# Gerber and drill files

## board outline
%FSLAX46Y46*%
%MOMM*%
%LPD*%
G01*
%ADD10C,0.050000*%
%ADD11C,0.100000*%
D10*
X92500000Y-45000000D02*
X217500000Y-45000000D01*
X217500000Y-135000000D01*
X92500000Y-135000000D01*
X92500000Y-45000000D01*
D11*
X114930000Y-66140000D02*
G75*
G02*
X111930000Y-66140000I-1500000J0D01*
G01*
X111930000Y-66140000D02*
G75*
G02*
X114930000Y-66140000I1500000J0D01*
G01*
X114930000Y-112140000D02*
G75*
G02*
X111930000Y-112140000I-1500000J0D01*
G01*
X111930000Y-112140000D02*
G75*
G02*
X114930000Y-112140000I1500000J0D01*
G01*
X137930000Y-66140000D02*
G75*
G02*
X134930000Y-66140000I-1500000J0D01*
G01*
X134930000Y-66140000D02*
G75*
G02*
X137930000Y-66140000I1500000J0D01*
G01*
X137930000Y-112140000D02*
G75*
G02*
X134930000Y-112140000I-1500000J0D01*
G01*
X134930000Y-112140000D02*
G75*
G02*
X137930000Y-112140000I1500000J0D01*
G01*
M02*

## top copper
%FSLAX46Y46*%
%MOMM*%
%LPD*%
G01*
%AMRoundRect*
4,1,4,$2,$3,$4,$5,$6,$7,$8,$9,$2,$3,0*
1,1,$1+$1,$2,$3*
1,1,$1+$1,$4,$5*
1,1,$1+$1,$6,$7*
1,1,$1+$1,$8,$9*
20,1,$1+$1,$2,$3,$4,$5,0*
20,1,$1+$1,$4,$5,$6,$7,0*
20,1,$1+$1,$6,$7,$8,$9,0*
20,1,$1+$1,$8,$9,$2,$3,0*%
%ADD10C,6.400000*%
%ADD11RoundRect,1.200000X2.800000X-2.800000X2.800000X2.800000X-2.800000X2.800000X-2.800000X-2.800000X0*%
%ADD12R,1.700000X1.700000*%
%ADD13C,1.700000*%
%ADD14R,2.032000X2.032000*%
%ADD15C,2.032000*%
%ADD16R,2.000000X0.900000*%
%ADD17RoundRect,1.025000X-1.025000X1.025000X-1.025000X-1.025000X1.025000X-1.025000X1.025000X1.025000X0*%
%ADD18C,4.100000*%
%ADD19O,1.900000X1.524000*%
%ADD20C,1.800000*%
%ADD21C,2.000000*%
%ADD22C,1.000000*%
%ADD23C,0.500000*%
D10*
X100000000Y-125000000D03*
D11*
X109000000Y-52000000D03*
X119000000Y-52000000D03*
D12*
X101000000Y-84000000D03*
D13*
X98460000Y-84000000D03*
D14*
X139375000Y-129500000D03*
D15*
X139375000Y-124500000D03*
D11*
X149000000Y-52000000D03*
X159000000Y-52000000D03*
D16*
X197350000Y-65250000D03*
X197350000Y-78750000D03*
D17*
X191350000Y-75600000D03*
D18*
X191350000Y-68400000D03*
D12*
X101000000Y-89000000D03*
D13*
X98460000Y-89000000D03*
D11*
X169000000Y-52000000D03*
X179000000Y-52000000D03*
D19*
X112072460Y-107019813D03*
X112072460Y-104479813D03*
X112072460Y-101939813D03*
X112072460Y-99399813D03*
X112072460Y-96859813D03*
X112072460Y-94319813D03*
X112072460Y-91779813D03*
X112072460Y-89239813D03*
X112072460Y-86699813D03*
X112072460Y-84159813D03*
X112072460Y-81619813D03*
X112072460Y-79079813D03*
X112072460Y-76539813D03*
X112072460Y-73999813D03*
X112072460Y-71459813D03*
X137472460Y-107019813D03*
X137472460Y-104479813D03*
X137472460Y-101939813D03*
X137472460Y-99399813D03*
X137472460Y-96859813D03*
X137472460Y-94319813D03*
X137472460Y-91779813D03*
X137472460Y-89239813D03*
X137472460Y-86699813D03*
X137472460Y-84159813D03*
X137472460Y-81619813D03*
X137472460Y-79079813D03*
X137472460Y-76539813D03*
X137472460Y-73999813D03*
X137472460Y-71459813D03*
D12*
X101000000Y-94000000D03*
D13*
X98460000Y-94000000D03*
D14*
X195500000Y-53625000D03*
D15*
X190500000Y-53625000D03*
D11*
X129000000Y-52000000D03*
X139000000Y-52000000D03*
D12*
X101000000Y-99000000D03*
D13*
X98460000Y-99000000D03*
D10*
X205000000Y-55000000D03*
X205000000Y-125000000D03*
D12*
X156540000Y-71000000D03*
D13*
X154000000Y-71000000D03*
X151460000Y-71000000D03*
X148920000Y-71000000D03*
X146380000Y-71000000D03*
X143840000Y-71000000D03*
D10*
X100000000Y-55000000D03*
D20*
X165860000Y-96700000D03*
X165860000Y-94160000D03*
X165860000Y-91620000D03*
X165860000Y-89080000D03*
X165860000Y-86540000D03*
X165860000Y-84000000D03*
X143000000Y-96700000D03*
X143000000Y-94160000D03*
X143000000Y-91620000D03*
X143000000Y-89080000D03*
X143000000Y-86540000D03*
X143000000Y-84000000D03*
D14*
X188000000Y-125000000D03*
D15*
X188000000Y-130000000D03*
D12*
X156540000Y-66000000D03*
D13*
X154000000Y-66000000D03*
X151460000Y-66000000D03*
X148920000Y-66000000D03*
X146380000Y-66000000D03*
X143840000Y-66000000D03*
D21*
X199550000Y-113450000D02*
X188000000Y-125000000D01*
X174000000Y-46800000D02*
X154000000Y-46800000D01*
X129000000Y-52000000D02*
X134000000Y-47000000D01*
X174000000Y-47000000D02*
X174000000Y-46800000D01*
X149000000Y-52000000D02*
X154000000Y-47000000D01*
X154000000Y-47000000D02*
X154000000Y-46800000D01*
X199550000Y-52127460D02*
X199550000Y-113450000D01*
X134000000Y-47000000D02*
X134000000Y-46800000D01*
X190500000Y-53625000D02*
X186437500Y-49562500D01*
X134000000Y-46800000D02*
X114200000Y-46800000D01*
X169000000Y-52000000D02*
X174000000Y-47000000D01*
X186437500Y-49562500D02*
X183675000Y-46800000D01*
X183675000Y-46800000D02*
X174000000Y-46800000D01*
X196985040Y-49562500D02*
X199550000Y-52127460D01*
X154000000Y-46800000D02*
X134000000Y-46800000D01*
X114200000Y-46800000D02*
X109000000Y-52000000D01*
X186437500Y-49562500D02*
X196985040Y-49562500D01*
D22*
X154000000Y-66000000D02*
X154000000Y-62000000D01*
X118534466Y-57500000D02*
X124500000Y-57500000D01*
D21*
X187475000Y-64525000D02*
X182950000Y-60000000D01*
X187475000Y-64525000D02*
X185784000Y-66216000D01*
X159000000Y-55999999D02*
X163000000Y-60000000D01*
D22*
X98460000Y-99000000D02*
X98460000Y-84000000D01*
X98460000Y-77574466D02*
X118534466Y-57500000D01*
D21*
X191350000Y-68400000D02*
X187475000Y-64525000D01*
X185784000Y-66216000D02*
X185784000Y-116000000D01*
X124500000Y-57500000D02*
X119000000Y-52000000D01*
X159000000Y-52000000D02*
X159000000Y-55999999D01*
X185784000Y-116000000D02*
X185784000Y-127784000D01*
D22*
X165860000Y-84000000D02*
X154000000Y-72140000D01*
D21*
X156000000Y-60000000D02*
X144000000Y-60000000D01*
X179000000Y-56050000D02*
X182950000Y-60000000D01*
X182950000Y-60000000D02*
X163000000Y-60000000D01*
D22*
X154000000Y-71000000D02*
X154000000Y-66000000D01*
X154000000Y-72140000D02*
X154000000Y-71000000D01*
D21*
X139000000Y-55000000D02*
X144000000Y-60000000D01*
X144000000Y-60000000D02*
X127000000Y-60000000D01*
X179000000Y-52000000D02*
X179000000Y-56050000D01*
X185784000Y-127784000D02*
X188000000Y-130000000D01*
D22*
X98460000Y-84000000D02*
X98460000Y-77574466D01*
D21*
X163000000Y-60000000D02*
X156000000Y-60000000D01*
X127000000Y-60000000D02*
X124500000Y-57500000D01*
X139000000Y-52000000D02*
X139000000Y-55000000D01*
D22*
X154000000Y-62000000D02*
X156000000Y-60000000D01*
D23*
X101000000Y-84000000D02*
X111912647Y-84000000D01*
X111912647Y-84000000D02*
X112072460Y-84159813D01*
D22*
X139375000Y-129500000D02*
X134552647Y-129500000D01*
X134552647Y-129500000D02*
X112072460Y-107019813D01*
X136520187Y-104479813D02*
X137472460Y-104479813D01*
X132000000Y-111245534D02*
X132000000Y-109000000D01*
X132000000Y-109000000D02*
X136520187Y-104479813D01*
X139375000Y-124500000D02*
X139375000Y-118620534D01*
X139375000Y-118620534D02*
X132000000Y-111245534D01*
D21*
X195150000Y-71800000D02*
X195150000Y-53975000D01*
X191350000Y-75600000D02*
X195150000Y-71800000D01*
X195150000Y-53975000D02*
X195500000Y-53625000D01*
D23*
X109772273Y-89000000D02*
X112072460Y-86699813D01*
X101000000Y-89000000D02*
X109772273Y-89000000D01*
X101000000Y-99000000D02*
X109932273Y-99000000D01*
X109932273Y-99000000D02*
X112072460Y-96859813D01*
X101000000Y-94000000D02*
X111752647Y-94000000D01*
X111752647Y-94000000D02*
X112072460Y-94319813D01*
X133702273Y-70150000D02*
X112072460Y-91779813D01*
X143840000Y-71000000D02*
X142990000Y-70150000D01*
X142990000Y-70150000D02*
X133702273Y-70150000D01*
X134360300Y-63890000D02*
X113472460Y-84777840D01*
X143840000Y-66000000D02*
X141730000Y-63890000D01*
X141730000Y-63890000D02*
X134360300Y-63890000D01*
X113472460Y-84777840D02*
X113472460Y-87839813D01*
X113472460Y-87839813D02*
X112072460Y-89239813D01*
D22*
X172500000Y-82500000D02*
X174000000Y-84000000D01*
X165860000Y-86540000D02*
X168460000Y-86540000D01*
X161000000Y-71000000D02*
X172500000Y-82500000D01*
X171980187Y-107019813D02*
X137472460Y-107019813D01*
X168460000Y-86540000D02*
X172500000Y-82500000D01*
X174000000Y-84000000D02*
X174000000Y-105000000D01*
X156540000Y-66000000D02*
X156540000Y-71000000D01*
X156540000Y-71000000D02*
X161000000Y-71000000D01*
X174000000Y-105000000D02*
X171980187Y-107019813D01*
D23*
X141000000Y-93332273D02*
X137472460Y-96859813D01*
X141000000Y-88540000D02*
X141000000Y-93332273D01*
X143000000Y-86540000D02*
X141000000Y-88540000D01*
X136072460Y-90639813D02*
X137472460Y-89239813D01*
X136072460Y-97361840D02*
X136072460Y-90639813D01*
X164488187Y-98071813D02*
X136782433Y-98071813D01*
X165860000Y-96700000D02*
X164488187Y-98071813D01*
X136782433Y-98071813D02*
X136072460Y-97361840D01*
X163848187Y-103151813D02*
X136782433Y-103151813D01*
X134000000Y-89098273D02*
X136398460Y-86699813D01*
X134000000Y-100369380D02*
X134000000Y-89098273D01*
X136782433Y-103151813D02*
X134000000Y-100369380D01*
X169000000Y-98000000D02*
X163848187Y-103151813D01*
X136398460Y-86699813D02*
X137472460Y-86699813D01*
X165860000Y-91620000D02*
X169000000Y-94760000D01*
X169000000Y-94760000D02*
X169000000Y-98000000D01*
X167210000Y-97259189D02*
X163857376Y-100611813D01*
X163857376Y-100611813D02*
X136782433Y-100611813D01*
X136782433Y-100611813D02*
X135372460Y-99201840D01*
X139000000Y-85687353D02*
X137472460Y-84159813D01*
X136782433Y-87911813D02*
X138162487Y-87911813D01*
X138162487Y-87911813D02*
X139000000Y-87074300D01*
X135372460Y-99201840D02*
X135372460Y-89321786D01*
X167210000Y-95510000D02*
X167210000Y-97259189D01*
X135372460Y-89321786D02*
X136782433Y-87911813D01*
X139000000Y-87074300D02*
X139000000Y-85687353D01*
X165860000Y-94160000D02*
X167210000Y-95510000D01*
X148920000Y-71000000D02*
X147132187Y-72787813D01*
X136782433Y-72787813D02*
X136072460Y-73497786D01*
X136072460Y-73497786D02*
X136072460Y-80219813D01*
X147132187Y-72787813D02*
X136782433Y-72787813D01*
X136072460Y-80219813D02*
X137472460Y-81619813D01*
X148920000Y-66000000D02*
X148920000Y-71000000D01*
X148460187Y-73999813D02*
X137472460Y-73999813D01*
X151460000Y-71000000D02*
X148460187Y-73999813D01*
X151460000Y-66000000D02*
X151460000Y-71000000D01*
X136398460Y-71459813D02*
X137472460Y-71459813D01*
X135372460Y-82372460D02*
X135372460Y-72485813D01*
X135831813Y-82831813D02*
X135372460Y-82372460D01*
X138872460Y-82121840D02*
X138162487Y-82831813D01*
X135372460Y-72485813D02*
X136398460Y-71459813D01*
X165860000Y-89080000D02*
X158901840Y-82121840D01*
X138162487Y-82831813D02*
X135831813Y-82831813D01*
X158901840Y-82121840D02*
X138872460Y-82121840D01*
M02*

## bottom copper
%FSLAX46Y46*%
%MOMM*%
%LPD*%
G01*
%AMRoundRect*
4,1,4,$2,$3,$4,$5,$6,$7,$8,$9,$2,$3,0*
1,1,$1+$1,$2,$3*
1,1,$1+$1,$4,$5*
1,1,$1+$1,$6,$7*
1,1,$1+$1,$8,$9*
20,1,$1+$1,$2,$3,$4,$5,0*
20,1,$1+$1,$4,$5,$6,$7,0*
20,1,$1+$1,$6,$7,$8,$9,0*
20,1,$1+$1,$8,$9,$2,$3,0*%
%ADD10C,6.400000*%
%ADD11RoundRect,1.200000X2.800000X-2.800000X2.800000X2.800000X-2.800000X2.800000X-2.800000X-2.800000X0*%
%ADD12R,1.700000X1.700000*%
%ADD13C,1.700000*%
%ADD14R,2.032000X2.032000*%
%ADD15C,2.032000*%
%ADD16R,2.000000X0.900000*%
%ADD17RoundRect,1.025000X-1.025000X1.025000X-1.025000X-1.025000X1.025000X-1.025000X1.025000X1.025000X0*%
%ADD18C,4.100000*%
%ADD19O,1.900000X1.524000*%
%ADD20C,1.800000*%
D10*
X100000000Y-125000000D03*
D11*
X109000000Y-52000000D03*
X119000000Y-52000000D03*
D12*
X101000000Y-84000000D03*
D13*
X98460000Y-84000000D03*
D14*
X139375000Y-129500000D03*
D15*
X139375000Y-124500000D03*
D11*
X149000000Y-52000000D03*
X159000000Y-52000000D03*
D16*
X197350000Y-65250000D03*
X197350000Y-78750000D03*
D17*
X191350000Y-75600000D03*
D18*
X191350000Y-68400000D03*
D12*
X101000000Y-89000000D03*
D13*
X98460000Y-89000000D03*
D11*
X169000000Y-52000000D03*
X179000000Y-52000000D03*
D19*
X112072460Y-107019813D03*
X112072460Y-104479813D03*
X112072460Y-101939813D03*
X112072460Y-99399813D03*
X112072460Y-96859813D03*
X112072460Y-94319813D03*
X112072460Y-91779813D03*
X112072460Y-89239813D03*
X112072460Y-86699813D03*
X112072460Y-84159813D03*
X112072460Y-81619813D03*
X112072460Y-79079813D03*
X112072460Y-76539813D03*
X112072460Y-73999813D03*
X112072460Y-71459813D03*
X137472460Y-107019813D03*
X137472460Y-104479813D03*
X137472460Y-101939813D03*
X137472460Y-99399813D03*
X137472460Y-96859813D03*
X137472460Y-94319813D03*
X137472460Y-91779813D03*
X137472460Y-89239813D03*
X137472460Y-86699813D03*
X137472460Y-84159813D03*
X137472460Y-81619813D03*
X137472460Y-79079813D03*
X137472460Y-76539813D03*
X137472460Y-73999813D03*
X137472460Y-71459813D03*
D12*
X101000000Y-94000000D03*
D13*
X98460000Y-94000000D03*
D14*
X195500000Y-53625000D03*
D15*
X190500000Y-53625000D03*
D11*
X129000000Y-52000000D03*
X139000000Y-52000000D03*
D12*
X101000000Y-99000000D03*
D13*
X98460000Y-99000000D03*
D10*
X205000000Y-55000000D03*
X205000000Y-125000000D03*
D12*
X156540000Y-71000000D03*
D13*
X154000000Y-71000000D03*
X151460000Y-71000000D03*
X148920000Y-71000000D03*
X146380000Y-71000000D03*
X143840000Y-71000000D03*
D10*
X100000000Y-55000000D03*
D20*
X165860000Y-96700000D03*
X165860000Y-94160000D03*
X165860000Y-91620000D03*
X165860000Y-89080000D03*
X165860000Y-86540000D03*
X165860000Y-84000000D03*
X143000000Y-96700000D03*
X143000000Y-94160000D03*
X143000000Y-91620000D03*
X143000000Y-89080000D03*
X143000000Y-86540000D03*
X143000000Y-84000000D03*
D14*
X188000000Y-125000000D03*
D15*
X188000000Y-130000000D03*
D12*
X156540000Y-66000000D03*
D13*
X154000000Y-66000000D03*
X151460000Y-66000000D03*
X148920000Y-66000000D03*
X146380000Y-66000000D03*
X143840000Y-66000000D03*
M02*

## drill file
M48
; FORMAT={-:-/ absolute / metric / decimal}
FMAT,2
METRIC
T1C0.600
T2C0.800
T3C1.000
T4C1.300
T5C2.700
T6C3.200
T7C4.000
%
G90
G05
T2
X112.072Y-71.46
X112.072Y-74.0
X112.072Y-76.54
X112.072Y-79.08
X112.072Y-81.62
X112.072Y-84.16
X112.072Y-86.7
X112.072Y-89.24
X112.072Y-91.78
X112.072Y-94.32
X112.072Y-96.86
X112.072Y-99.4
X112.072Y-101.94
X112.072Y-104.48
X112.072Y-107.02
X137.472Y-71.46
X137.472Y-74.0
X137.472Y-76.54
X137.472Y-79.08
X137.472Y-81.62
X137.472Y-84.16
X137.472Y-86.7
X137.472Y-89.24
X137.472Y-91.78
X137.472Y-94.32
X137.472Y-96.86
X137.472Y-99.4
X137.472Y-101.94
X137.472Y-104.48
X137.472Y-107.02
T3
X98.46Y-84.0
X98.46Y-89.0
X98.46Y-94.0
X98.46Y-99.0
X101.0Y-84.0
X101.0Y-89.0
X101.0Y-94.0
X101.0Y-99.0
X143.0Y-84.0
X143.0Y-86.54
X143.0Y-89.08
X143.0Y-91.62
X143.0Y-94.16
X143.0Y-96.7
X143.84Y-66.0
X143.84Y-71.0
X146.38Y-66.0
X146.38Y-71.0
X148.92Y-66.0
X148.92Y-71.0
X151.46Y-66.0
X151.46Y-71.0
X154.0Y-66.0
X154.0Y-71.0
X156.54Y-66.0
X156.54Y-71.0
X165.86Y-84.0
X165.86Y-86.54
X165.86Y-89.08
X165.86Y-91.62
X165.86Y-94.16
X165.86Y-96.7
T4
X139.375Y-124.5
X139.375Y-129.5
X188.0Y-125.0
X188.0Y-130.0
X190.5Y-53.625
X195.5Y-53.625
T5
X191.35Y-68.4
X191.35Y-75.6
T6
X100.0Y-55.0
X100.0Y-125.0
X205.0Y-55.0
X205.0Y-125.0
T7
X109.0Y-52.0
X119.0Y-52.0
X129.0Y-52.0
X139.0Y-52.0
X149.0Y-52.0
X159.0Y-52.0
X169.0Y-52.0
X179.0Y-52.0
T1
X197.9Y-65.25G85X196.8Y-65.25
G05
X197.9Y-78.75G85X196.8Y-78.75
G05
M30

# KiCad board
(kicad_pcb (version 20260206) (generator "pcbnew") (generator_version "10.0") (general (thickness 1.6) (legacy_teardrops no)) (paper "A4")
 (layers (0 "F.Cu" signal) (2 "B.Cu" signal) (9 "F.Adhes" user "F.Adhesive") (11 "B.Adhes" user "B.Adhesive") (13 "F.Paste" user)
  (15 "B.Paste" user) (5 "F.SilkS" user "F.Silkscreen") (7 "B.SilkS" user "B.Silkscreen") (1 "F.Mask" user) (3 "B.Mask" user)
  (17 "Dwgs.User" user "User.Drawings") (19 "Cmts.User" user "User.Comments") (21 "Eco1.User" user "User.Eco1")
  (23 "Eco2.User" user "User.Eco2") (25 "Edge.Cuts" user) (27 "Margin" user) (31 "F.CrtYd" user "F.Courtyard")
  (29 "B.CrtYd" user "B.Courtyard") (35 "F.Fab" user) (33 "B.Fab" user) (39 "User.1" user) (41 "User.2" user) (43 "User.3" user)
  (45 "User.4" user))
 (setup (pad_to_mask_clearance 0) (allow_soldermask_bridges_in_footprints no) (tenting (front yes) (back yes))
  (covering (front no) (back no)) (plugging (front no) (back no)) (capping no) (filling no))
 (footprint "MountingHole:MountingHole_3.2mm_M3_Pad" (layer "F.Cu") (at 100 125)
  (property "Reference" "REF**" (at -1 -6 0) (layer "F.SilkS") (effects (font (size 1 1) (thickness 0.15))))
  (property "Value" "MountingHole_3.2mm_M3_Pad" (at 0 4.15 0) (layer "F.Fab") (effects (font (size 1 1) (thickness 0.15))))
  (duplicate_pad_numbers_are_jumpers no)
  (pad "1" thru_hole circle (at 0 0) (size 6.4 6.4) (drill 3.2) (layers "*.Cu" "*.Mask") (remove_unused_layers no) (zone_connect 2)))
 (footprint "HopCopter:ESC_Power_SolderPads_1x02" (layer "F.Cu") (at 114 52)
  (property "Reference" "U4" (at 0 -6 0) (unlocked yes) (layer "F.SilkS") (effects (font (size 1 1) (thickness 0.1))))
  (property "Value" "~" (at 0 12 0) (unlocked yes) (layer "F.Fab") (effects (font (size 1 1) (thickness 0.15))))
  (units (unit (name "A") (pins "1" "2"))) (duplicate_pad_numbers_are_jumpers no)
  (pad "1" thru_hole roundrect (at -5 0 90) (size 8 8) (drill 4) (layers "*.Cu" "*.Mask") (remove_unused_layers no) (roundrect_rratio 0.15)
   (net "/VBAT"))
  (pad "2" thru_hole roundrect (at 5 0 90) (size 8 8) (drill 4) (layers "*.Cu" "*.Mask") (remove_unused_layers no) (roundrect_rratio 0.15)
   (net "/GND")))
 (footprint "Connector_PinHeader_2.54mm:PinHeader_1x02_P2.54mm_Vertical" (layer "F.Cu") (at 101 84 -90)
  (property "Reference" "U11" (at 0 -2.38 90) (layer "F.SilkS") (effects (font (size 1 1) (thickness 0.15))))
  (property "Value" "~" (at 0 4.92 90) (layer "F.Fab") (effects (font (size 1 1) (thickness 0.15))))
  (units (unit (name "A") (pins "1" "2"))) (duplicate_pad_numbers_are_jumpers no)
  (pad "1" thru_hole rect (at 0 0 270) (size 1.7 1.7) (drill 1) (layers "*.Cu" "*.Mask") (remove_unused_layers no) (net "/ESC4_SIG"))
  (pad "2" thru_hole circle (at 0 2.54 270) (size 1.7 1.7) (drill 1) (layers "*.Cu" "*.Mask") (remove_unused_layers no) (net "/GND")))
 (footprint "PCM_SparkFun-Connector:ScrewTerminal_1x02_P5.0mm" (layer "F.Cu") (at 139.375 129.5 90)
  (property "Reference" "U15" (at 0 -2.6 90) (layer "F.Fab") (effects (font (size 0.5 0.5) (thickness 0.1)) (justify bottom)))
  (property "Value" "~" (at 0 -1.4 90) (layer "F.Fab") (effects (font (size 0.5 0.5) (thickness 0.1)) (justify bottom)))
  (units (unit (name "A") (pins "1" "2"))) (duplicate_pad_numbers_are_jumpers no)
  (pad "1" thru_hole rect (at 0 0 90) (size 2.032 2.032) (drill 1.3) (layers "*.Cu" "*.Mask") (remove_unused_layers no)
   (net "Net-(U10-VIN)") (thermal_bridge_angle 0))
  (pad "2" thru_hole circle (at 5 0 90) (size 2.032 2.032) (drill 1.3) (layers "*.Cu" "*.Mask") (remove_unused_layers no)
   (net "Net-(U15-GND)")))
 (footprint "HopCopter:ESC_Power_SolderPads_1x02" (layer "F.Cu") (at 154 52)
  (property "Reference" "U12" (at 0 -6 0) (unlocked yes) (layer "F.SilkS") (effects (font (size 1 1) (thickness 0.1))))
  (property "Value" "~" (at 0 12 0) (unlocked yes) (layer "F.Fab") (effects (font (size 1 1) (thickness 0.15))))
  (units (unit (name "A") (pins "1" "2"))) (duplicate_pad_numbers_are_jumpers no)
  (pad "1" thru_hole roundrect (at -5 0 90) (size 8 8) (drill 4) (layers "*.Cu" "*.Mask") (remove_unused_layers no) (roundrect_rratio 0.15)
   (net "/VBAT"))
  (pad "2" thru_hole roundrect (at 5 0 90) (size 8 8) (drill 4) (layers "*.Cu" "*.Mask") (remove_unused_layers no) (roundrect_rratio 0.15)
   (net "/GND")))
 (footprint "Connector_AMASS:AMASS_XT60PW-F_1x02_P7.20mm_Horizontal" (layer "F.Cu") (at 191.35 75.6 -90)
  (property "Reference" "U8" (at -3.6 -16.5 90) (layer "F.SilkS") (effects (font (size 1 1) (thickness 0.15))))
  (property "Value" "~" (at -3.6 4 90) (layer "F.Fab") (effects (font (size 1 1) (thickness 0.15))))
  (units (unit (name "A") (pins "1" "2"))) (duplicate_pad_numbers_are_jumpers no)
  (pad "" thru_hole rect (at -10.35 -6 270) (size 0.9 2) (drill oval 0.6 1.7) (layers "*.Cu" "*.Mask") (remove_unused_layers no))
  (pad "" thru_hole rect (at 3.15 -6 270) (size 0.9 2) (drill oval 0.6 1.7) (layers "*.Cu" "*.Mask") (remove_unused_layers no))
  (pad "1" thru_hole roundrect (at 0 0 270) (size 4.1 4.1) (drill 2.7) (layers "*.Cu" "*.Mask") (remove_unused_layers no)
   (roundrect_rratio 0.25) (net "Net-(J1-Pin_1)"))
  (pad "2" thru_hole circle (at -7.2 0 270) (size 4.1 4.1) (drill 2.7) (layers "*.Cu" "*.Mask") (remove_unused_layers no) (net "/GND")))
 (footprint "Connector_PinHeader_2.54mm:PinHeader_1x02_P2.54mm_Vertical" (layer "F.Cu") (at 101 89 -90)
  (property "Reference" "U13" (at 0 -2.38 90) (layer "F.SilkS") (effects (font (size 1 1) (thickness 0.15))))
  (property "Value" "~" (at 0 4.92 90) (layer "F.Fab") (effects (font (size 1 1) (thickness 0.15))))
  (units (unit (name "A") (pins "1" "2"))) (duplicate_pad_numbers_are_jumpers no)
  (pad "1" thru_hole rect (at 0 0 270) (size 1.7 1.7) (drill 1) (layers "*.Cu" "*.Mask") (remove_unused_layers no) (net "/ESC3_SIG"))
  (pad "2" thru_hole circle (at 0 2.54 270) (size 1.7 1.7) (drill 1) (layers "*.Cu" "*.Mask") (remove_unused_layers no) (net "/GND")))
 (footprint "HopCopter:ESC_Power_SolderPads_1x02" (layer "F.Cu") (at 174 52)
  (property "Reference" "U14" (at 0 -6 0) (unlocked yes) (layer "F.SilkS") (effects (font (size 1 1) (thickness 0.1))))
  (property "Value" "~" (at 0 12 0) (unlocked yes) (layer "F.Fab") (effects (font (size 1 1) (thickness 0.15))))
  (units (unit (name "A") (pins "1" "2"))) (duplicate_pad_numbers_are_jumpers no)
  (pad "1" thru_hole roundrect (at -5 0 90) (size 8 8) (drill 4) (layers "*.Cu" "*.Mask") (remove_unused_layers no) (roundrect_rratio 0.15)
   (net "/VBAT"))
  (pad "2" thru_hole roundrect (at 5 0 90) (size 8 8) (drill 4) (layers "*.Cu" "*.Mask") (remove_unused_layers no) (roundrect_rratio 0.15)
   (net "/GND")))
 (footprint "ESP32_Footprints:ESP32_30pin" (layer "F.Cu") (at 124 90)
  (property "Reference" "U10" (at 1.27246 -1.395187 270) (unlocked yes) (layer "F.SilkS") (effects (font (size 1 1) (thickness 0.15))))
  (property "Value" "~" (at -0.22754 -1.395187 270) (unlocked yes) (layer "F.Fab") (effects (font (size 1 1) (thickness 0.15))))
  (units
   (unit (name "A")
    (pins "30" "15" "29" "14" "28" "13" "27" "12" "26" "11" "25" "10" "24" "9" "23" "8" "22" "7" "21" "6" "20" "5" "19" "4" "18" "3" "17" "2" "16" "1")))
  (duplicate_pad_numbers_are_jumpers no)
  (fp_circle (center -10.57 -23.86) (end -10.57 -22.36) (stroke (width 0.1) (type default)) (fill no) (layer "Edge.Cuts"))
  (fp_circle (center -10.57 22.14) (end -10.57 23.64) (stroke (width 0.1) (type default)) (fill no) (layer "Edge.Cuts"))
  (fp_circle (center 12.43 -23.86) (end 12.43 -22.36) (stroke (width 0.1) (type default)) (fill no) (layer "Edge.Cuts"))
  (fp_circle (center 12.43 22.14) (end 12.43 23.64) (stroke (width 0.1) (type default)) (fill no) (layer "Edge.Cuts"))
  (pad "1" thru_hole oval (at -11.92754 17.019813 270) (size 1.524 1.9) (drill 0.8) (layers "*.Cu" "*.Mask") (remove_unused_layers no)
   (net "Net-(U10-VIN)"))
  (pad "2" thru_hole oval (at -11.92754 14.479813 270) (size 1.524 1.9) (drill 0.8) (layers "*.Cu" "*.Mask") (remove_unused_layers no)
   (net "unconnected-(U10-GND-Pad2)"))
  (pad "3" thru_hole oval (at -11.92754 11.939813 270) (size 1.524 1.9) (drill 0.8) (layers "*.Cu" "*.Mask") (remove_unused_layers no)
   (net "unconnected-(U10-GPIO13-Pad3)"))
  (pad "4" thru_hole oval (at -11.92754 9.399813 270) (size 1.524 1.9) (drill 0.8) (layers "*.Cu" "*.Mask") (remove_unused_layers no)
   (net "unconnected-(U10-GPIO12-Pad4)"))
  (pad "5" thru_hole oval (at -11.92754 6.859813 270) (size 1.524 1.9) (drill 0.8) (layers "*.Cu" "*.Mask") (remove_unused_layers no)
   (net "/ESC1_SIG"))
  (pad "6" thru_hole oval (at -11.92754 4.319813 270) (size 1.524 1.9) (drill 0.8) (layers "*.Cu" "*.Mask") (remove_unused_layers no)
   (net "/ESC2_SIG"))
  (pad "7" thru_hole oval (at -11.92754 1.779813 270) (size 1.524 1.9) (drill 0.8) (layers "*.Cu" "*.Mask") (remove_unused_layers no)
   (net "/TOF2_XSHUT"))
  (pad "8" thru_hole oval (at -11.92754 -0.760187 270) (size 1.524 1.9) (drill 0.8) (layers "*.Cu" "*.Mask") (remove_unused_layers no)
   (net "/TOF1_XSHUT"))
  (pad "9" thru_hole oval (at -11.92754 -3.300187 270) (size 1.524 1.9) (drill 0.8) (layers "*.Cu" "*.Mask") (remove_unused_layers no)
   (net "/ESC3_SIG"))
  (pad "10" thru_hole oval (at -11.92754 -5.840187 270) (size 1.524 1.9) (drill 0.8) (layers "*.Cu" "*.Mask") (remove_unused_layers no)
   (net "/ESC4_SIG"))
  (pad "11" thru_hole oval (at -11.92754 -8.380187 270) (size 1.524 1.9) (drill 0.8) (layers "*.Cu" "*.Mask") (remove_unused_layers no)
   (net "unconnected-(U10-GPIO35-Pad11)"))
  (pad "12" thru_hole oval (at -11.92754 -10.920187 270) (size 1.524 1.9) (drill 0.8) (layers "*.Cu" "*.Mask") (remove_unused_layers no)
   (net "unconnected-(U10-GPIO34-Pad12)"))
  (pad "13" thru_hole oval (at -11.92754 -13.460187 270) (size 1.524 1.9) (drill 0.8) (layers "*.Cu" "*.Mask") (remove_unused_layers no)
   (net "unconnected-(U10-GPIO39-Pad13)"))
  (pad "14" thru_hole oval (at -11.92754 -16.000187 270) (size 1.524 1.9) (drill 0.8) (layers "*.Cu" "*.Mask") (remove_unused_layers no)
   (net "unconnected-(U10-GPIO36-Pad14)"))
  (pad "15" thru_hole oval (at -11.92754 -18.540187 270) (size 1.524 1.9) (drill 0.8) (layers "*.Cu" "*.Mask") (remove_unused_layers no)
   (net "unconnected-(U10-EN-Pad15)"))
  (pad "16" thru_hole oval (at 13.47246 17.019813 270) (size 1.524 1.9) (drill 0.8) (layers "*.Cu" "*.Mask") (remove_unused_layers no)
   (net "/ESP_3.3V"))
  (pad "17" thru_hole oval (at 13.47246 14.479813 270) (size 1.524 1.9) (drill 0.8) (layers "*.Cu" "*.Mask") (remove_unused_layers no)
   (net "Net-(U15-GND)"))
  (pad "18" thru_hole oval (at 13.47246 11.939813 270) (size 1.524 1.9) (drill 0.8) (layers "*.Cu" "*.Mask") (remove_unused_layers no)
   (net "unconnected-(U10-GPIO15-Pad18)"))
  (pad "19" thru_hole oval (at 13.47246 9.399813 270) (size 1.524 1.9) (drill 0.8) (layers "*.Cu" "*.Mask") (remove_unused_layers no)
   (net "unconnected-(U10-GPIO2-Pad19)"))
  (pad "20" thru_hole oval (at 13.47246 6.859813 270) (size 1.524 1.9) (drill 0.8) (layers "*.Cu" "*.Mask" "Dwgs.User")
   (remove_unused_layers no) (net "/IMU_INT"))
  (pad "21" thru_hole oval (at 13.47246 4.319813 270) (size 1.524 1.9) (drill 0.8) (layers "*.Cu" "*.Mask") (remove_unused_layers no)
   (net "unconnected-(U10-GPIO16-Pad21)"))
  (pad "22" thru_hole oval (at 13.47246 1.779813 270) (size 1.524 1.9) (drill 0.8) (layers "*.Cu" "*.Mask") (remove_unused_layers no)
   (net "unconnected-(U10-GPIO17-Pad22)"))
  (pad "23" thru_hole oval (at 13.47246 -0.760187 270) (size 1.524 1.9) (drill 0.8) (layers "*.Cu" "*.Mask") (remove_unused_layers no)
   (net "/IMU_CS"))
  (pad "24" thru_hole oval (at 13.47246 -3.300187 270) (size 1.524 1.9) (drill 0.8) (layers "*.Cu" "*.Mask") (remove_unused_layers no)
   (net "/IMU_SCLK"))
  (pad "25" thru_hole oval (at 13.47246 -5.840187 270) (size 1.524 1.9) (drill 0.8) (layers "*.Cu" "*.Mask") (remove_unused_layers no)
   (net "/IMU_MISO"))
  (pad "26" thru_hole oval (at 13.47246 -8.380187 270) (size 1.524 1.9) (drill 0.8) (layers "*.Cu" "*.Mask") (remove_unused_layers no)
   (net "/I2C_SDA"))
  (pad "27" thru_hole oval (at 13.47246 -10.920187 270) (size 1.524 1.9) (drill 0.8) (layers "*.Cu" "*.Mask") (remove_unused_layers no)
   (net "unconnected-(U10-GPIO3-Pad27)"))
  (pad "28" thru_hole oval (at 13.47246 -13.460187 270) (size 1.524 1.9) (drill 0.8) (layers "*.Cu" "*.Mask") (remove_unused_layers no)
   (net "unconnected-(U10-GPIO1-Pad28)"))
  (pad "29" thru_hole oval (at 13.47246 -16.000187 270) (size 1.524 1.9) (drill 0.8) (layers "*.Cu" "*.Mask") (remove_unused_layers no)
   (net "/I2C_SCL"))
  (pad "30" thru_hole oval (at 13.47246 -18.540187 270) (size 1.524 1.9) (drill 0.8) (layers "*.Cu" "*.Mask") (remove_unused_layers no)
   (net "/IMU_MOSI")))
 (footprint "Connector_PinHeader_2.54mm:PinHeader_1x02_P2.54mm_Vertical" (layer "F.Cu") (at 101 94 -90)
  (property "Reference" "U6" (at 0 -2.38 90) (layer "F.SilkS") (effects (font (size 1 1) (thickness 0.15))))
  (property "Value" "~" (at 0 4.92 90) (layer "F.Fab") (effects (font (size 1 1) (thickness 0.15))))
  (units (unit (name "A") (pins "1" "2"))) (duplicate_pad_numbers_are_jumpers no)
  (pad "1" thru_hole rect (at 0 0 270) (size 1.7 1.7) (drill 1) (layers "*.Cu" "*.Mask") (remove_unused_layers no) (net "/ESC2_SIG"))
  (pad "2" thru_hole circle (at 0 2.54 270) (size 1.7 1.7) (drill 1) (layers "*.Cu" "*.Mask") (remove_unused_layers no) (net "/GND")))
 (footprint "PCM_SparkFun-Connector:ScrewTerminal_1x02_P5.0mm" (layer "F.Cu") (at 195.5 53.625 180)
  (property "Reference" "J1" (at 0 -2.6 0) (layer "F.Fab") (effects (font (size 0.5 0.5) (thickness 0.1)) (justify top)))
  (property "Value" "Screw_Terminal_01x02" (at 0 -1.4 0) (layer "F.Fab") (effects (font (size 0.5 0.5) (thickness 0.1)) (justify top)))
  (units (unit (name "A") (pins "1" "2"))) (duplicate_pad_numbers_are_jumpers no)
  (pad "1" thru_hole rect (at 0 0 180) (size 2.032 2.032) (drill 1.3) (layers "*.Cu" "*.Mask") (remove_unused_layers no)
   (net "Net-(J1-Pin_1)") (thermal_bridge_angle 0))
  (pad "2" thru_hole circle (at 5 0 180) (size 2.032 2.032) (drill 1.3) (layers "*.Cu" "*.Mask") (remove_unused_layers no) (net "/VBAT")))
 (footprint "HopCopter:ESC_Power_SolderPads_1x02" (layer "F.Cu") (at 134 52)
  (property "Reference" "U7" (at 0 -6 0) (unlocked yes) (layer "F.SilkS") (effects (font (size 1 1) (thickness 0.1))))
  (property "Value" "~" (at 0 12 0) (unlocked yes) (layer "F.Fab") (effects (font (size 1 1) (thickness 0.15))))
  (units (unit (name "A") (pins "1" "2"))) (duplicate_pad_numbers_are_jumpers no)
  (pad "1" thru_hole roundrect (at -5 0 90) (size 8 8) (drill 4) (layers "*.Cu" "*.Mask") (remove_unused_layers no) (roundrect_rratio 0.15)
   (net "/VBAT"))
  (pad "2" thru_hole roundrect (at 5 0 90) (size 8 8) (drill 4) (layers "*.Cu" "*.Mask") (remove_unused_layers no) (roundrect_rratio 0.15)
   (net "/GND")))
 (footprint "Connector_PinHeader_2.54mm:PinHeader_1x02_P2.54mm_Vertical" (layer "F.Cu") (at 101 99 -90)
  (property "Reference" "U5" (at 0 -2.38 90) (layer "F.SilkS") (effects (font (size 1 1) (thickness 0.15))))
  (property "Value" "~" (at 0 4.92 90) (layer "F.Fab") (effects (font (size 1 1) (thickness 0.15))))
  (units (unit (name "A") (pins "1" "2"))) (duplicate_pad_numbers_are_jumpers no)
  (pad "1" thru_hole rect (at 0 0 270) (size 1.7 1.7) (drill 1) (layers "*.Cu" "*.Mask") (remove_unused_layers no) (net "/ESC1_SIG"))
  (pad "2" thru_hole circle (at 0 2.54 270) (size 1.7 1.7) (drill 1) (layers "*.Cu" "*.Mask") (remove_unused_layers no) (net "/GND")))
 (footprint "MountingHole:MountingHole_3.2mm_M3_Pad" (layer "F.Cu") (at 205 55)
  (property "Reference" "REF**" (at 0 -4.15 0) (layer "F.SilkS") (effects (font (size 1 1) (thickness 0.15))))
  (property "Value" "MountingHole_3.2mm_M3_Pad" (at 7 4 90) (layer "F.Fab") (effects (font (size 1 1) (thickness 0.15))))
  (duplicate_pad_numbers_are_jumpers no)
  (pad "1" thru_hole circle (at 0 0) (size 6.4 6.4) (drill 3.2) (layers "*.Cu" "*.Mask") (remove_unused_layers no) (zone_connect 2)))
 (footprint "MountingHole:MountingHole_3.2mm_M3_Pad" (layer "F.Cu") (at 205 125)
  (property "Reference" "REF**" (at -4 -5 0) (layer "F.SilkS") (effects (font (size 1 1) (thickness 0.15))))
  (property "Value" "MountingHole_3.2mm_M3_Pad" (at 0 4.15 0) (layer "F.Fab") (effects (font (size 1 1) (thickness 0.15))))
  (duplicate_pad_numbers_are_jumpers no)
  (pad "1" thru_hole circle (at 0 0) (size 6.4 6.4) (drill 3.2) (layers "*.Cu" "*.Mask") (remove_unused_layers no) (zone_connect 2)))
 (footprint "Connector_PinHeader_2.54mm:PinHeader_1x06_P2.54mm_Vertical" (layer "F.Cu") (at 156.54 71 -90)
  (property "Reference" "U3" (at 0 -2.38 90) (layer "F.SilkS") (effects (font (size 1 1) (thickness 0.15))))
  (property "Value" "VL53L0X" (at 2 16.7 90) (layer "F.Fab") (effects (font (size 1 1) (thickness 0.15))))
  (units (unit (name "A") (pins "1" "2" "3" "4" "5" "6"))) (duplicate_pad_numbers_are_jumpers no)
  (pad "1" thru_hole rect (at 0 0 270) (size 1.7 1.7) (drill 1) (layers "*.Cu" "*.Mask") (remove_unused_layers no) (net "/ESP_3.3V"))
  (pad "2" thru_hole circle (at 0 2.54 270) (size 1.7 1.7) (drill 1) (layers "*.Cu" "*.Mask") (remove_unused_layers no) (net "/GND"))
  (pad "3" thru_hole circle (at 0 5.08 270) (size 1.7 1.7) (drill 1) (layers "*.Cu" "*.Mask") (remove_unused_layers no) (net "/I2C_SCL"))
  (pad "4" thru_hole circle (at 0 7.62 270) (size 1.7 1.7) (drill 1) (layers "*.Cu" "*.Mask") (remove_unused_layers no) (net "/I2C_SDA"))
  (pad "5" thru_hole circle (at 0 10.16 270) (size 1.7 1.7) (drill 1) (layers "*.Cu" "*.Mask") (remove_unused_layers no)
   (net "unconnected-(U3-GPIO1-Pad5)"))
  (pad "6" thru_hole circle (at 0 12.7 270) (size 1.7 1.7) (drill 1) (layers "*.Cu" "*.Mask") (remove_unused_layers no) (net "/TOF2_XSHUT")))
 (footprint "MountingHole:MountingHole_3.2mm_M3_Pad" (layer "F.Cu") (at 100 55)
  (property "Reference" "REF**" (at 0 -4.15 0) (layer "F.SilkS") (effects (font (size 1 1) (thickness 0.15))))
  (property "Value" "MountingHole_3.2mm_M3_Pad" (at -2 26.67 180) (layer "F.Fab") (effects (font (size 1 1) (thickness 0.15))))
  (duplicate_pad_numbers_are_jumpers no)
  (pad "1" thru_hole circle (at 0 0) (size 6.4 6.4) (drill 3.2) (layers "*.Cu" "*.Mask") (remove_unused_layers no) (zone_connect 2)))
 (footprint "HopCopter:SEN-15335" (layer "F.Cu") (at 165.86 96.7 180)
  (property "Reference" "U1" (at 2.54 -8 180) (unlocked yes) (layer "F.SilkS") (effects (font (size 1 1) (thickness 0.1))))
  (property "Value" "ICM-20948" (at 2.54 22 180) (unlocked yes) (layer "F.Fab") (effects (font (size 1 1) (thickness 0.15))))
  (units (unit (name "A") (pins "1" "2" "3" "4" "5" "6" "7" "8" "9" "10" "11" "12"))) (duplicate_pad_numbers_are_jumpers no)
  (pad "1" thru_hole circle (at 0 0 180) (size 1.8 1.8) (drill 1) (layers "*.Cu" "*.Mask") (remove_unused_layers no) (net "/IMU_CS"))
  (pad "2" thru_hole circle (at 0 2.54 180) (size 1.8 1.8) (drill 1) (layers "*.Cu" "*.Mask" "Eco1.User") (remove_unused_layers no)
   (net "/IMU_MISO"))
  (pad "3" thru_hole circle (at 0 5.08 180) (size 1.8 1.8) (drill 1) (layers "*.Cu" "*.Mask" "Eco1.User") (remove_unused_layers no)
   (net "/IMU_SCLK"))
  (pad "4" thru_hole circle (at 0 7.62 180) (size 1.8 1.8) (drill 1) (layers "*.Cu" "*.Mask" "Eco1.User") (remove_unused_layers no)
   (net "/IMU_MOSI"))
  (pad "5" thru_hole circle (at 0 10.16 180) (size 1.8 1.8) (drill 1) (layers "*.Cu" "*.Mask" "Eco1.User") (remove_unused_layers no)
   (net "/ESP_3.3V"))
  (pad "6" thru_hole circle (at 0 12.7 180) (size 1.8 1.8) (drill 1) (layers "*.Cu" "*.Mask" "Eco1.User") (remove_unused_layers no)
   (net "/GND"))
  (pad "7" thru_hole circle (at 22.86 0 180) (size 1.8 1.8) (drill 1) (layers "*.Cu" "*.Mask") (remove_unused_layers no)
   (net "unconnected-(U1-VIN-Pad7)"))
  (pad "8" thru_hole circle (at 22.86 2.54 180) (size 1.8 1.8) (drill 1) (layers "*.Cu" "*.Mask" "Eco1.User") (remove_unused_layers no)
   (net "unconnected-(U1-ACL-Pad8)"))
  (pad "9" thru_hole circle (at 22.86 5.08 180) (size 1.8 1.8) (drill 1) (layers "*.Cu" "*.Mask" "Eco1.User") (remove_unused_layers no)
   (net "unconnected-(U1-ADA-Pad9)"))
  (pad "10" thru_hole circle (at 22.86 7.62 180) (size 1.8 1.8) (drill 1) (layers "*.Cu" "*.Mask" "Eco1.User") (remove_unused_layers no)
   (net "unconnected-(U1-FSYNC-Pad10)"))
  (pad "11" thru_hole circle (at 22.86 10.16 180) (size 1.8 1.8) (drill 1) (layers "*.Cu" "*.Mask" "Eco1.User") (remove_unused_layers no)
   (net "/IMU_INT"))
  (pad "12" thru_hole circle (at 22.86 12.7 180) (size 1.8 1.8) (drill 1) (layers "*.Cu" "*.Mask" "Eco1.User") (remove_unused_layers no)
   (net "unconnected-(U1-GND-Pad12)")))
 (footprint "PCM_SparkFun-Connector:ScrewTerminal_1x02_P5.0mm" (layer "F.Cu") (at 188 125 -90)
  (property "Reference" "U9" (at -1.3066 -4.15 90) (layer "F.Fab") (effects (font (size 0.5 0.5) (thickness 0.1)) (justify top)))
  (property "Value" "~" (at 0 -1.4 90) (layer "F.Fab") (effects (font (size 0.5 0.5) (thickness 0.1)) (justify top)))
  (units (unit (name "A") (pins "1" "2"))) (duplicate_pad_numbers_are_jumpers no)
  (pad "1" thru_hole rect (at 0 0 270) (size 2.032 2.032) (drill 1.3) (layers "*.Cu" "*.Mask") (remove_unused_layers no) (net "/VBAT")
   (thermal_bridge_angle 0))
  (pad "2" thru_hole circle (at 5 0 270) (size 2.032 2.032) (drill 1.3) (layers "*.Cu" "*.Mask") (remove_unused_layers no) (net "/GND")))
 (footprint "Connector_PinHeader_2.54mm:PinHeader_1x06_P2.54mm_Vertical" (layer "F.Cu") (at 156.54 66 -90)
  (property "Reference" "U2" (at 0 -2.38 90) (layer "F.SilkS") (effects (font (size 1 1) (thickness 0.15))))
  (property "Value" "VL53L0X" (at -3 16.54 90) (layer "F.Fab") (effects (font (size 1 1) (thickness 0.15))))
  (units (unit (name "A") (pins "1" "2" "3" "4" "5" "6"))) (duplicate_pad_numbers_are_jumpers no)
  (pad "1" thru_hole rect (at 0 0 270) (size 1.7 1.7) (drill 1) (layers "*.Cu" "*.Mask") (remove_unused_layers no) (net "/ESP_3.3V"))
  (pad "2" thru_hole circle (at 0 2.54 270) (size 1.7 1.7) (drill 1) (layers "*.Cu" "*.Mask") (remove_unused_layers no) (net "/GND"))
  (pad "3" thru_hole circle (at 0 5.08 270) (size 1.7 1.7) (drill 1) (layers "*.Cu" "*.Mask") (remove_unused_layers no) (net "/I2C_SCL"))
  (pad "4" thru_hole circle (at 0 7.62 270) (size 1.7 1.7) (drill 1) (layers "*.Cu" "*.Mask") (remove_unused_layers no) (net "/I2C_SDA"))
  (pad "5" thru_hole circle (at 0 10.16 270) (size 1.7 1.7) (drill 1) (layers "*.Cu" "*.Mask") (remove_unused_layers no)
   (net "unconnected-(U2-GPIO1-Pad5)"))
  (pad "6" thru_hole circle (at 0 12.7 270) (size 1.7 1.7) (drill 1) (layers "*.Cu" "*.Mask") (remove_unused_layers no) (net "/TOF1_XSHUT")))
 (gr_rect (start 92.5 45) (end 217.5 135) (stroke (width 0.05) (type solid)) (fill no) (layer "Edge.Cuts"))
 (segment (start 199.55 113.45) (end 188 125) (width 2) (layer "F.Cu") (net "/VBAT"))
 (segment (start 174 46.8) (end 154 46.8) (width 2) (layer "F.Cu") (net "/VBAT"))
 (segment (start 129 52) (end 134 47) (width 2) (layer "F.Cu") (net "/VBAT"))
 (segment (start 174 47) (end 174 46.8) (width 2) (layer "F.Cu") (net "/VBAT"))
 (segment (start 149 52) (end 154 47) (width 2) (layer "F.Cu") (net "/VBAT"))
 (segment (start 154 47) (end 154 46.8) (width 2) (layer "F.Cu") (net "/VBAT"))
 (segment (start 199.55 52.12746) (end 199.55 113.45) (width 2) (layer "F.Cu") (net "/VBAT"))
 (segment (start 134 47) (end 134 46.8) (width 2) (layer "F.Cu") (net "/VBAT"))
 (segment (start 190.5 53.625) (end 186.4375 49.5625) (width 2) (layer "F.Cu") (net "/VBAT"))
 (segment (start 134 46.8) (end 114.2 46.8) (width 2) (layer "F.Cu") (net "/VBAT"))
 (segment (start 169 52) (end 174 47) (width 2) (layer "F.Cu") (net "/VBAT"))
 (segment (start 186.4375 49.5625) (end 183.675 46.8) (width 2) (layer "F.Cu") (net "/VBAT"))
 (segment (start 183.675 46.8) (end 174 46.8) (width 2) (layer "F.Cu") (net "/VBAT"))
 (segment (start 196.98504 49.5625) (end 199.55 52.12746) (width 2) (layer "F.Cu") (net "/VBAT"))
 (segment (start 154 46.8) (end 134 46.8) (width 2) (layer "F.Cu") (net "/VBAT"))
 (segment (start 114.2 46.8) (end 109 52) (width 2) (layer "F.Cu") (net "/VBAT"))
 (segment (start 186.4375 49.5625) (end 196.98504 49.5625) (width 2) (layer "F.Cu") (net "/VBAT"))
 (segment (start 154 66) (end 154 62) (width 1) (layer "F.Cu") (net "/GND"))
 (segment (start 118.534466 57.5) (end 124.5 57.5) (width 1) (layer "F.Cu") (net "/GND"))
 (segment (start 187.475 64.525) (end 182.95 60) (width 2) (layer "F.Cu") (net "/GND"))
 (segment (start 187.475 64.525) (end 185.784 66.216) (width 2) (layer "F.Cu") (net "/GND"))
 (segment (start 159 55.999999) (end 163 60) (width 2) (layer "F.Cu") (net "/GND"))
 (segment (start 98.46 99) (end 98.46 84) (width 1) (layer "F.Cu") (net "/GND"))
 (segment (start 98.46 77.574466) (end 118.534466 57.5) (width 1) (layer "F.Cu") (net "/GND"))
 (segment (start 191.35 68.4) (end 187.475 64.525) (width 2) (layer "F.Cu") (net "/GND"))
 (segment (start 185.784 66.216) (end 185.784 116) (width 2) (layer "F.Cu") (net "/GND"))
 (segment (start 124.5 57.5) (end 119 52) (width 2) (layer "F.Cu") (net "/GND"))
 (segment (start 159 52) (end 159 55.999999) (width 2) (layer "F.Cu") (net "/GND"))
 (segment (start 185.784 116) (end 185.784 127.784) (width 2) (layer "F.Cu") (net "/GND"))
 (segment (start 165.86 84) (end 154 72.14) (width 1) (layer "F.Cu") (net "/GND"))
 (segment (start 156 60) (end 144 60) (width 2) (layer "F.Cu") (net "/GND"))
 (segment (start 179 56.05) (end 182.95 60) (width 2) (layer "F.Cu") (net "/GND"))
 (segment (start 182.95 60) (end 163 60) (width 2) (layer "F.Cu") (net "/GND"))
 (segment (start 154 71) (end 154 66) (width 1) (layer "F.Cu") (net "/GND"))
 (segment (start 154 72.14) (end 154 71) (width 1) (layer "F.Cu") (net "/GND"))
 (segment (start 139 55) (end 144 60) (width 2) (layer "F.Cu") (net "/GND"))
 (segment (start 144 60) (end 127 60) (width 2) (layer "F.Cu") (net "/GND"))
 (segment (start 179 52) (end 179 56.05) (width 2) (layer "F.Cu") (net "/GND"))
 (segment (start 185.784 127.784) (end 188 130) (width 2) (layer "F.Cu") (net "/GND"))
 (segment (start 98.46 84) (end 98.46 77.574466) (width 1) (layer "F.Cu") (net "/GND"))
 (segment (start 163 60) (end 156 60) (width 2) (layer "F.Cu") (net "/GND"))
 (segment (start 127 60) (end 124.5 57.5) (width 2) (layer "F.Cu") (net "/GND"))
 (segment (start 139 52) (end 139 55) (width 2) (layer "F.Cu") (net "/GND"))
 (segment (start 154 62) (end 156 60) (width 1) (layer "F.Cu") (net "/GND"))
 (segment (start 101 84) (end 111.912647 84) (width 0.5) (layer "F.Cu") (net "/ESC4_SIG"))
 (segment (start 111.912647 84) (end 112.07246 84.159813) (width 0.5) (layer "F.Cu") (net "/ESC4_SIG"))
 (segment (start 139.375 129.5) (end 134.552647 129.5) (width 1) (layer "F.Cu") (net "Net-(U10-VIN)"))
 (segment (start 134.552647 129.5) (end 112.07246 107.019813) (width 1) (layer "F.Cu") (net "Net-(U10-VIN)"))
 (segment (start 136.520187 104.479813) (end 137.47246 104.479813) (width 1) (layer "F.Cu") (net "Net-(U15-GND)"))
 (segment (start 132 111.245534) (end 132 109) (width 1) (layer "F.Cu") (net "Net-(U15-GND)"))
 (segment (start 132 109) (end 136.520187 104.479813) (width 1) (layer "F.Cu") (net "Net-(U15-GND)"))
 (segment (start 139.375 124.5) (end 139.375 118.620534) (width 1) (layer "F.Cu") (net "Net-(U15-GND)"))
 (segment (start 139.375 118.620534) (end 132 111.245534) (width 1) (layer "F.Cu") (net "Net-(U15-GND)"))
 (segment (start 195.15 71.8) (end 195.15 53.975) (width 2) (layer "F.Cu") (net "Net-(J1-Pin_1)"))
 (segment (start 191.35 75.6) (end 195.15 71.8) (width 2) (layer "F.Cu") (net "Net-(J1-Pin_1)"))
 (segment (start 195.15 53.975) (end 195.5 53.625) (width 2) (layer "F.Cu") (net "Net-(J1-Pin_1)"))
 (segment (start 109.772273 89) (end 112.07246 86.699813) (width 0.5) (layer "F.Cu") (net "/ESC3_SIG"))
 (segment (start 101 89) (end 109.772273 89) (width 0.5) (layer "F.Cu") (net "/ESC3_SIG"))
 (segment (start 101 99) (end 109.932273 99) (width 0.5) (layer "F.Cu") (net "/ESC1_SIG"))
 (segment (start 109.932273 99) (end 112.07246 96.859813) (width 0.5) (layer "F.Cu") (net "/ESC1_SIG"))
 (segment (start 101 94) (end 111.752647 94) (width 0.5) (layer "F.Cu") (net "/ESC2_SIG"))
 (segment (start 111.752647 94) (end 112.07246 94.319813) (width 0.5) (layer "F.Cu") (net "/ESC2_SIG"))
 (segment (start 133.702273 70.15) (end 112.07246 91.779813) (width 0.5) (layer "F.Cu") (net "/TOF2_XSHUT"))
 (segment (start 143.84 71) (end 142.99 70.15) (width 0.5) (layer "F.Cu") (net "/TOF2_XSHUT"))
 (segment (start 142.99 70.15) (end 133.702273 70.15) (width 0.5) (layer "F.Cu") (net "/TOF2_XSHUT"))
 (segment (start 134.3603 63.89) (end 113.47246 84.77784) (width 0.5) (layer "F.Cu") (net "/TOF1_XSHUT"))
 (segment (start 143.84 66) (end 141.73 63.89) (width 0.5) (layer "F.Cu") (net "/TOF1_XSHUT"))
 (segment (start 141.73 63.89) (end 134.3603 63.89) (width 0.5) (layer "F.Cu") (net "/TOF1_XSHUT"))
 (segment (start 113.47246 84.77784) (end 113.47246 87.839813) (width 0.5) (layer "F.Cu") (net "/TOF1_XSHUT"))
 (segment (start 113.47246 87.839813) (end 112.07246 89.239813) (width 0.5) (layer "F.Cu") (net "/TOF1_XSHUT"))
 (segment (start 172.5 82.5) (end 174 84) (width 1) (layer "F.Cu") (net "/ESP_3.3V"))
 (segment (start 165.86 86.54) (end 168.46 86.54) (width 1) (layer "F.Cu") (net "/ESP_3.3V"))
 (segment (start 161 71) (end 172.5 82.5) (width 1) (layer "F.Cu") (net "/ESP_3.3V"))
 (segment (start 171.980187 107.019813) (end 137.47246 107.019813) (width 1) (layer "F.Cu") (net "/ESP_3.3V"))
 (segment (start 168.46 86.54) (end 172.5 82.5) (width 1) (layer "F.Cu") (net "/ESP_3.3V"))
 (segment (start 174 84) (end 174 105) (width 1) (layer "F.Cu") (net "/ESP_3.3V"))
 (segment (start 156.54 66) (end 156.54 71) (width 1) (layer "F.Cu") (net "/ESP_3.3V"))
 (segment (start 156.54 71) (end 161 71) (width 1) (layer "F.Cu") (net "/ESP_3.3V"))
 (segment (start 174 105) (end 171.980187 107.019813) (width 1) (layer "F.Cu") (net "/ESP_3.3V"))
 (segment (start 141 93.332273) (end 137.47246 96.859813) (width 0.5) (layer "F.Cu") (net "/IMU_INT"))
 (segment (start 141 88.54) (end 141 93.332273) (width 0.5) (layer "F.Cu") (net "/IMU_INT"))
 (segment (start 143 86.54) (end 141 88.54) (width 0.5) (layer "F.Cu") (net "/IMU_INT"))
 (segment (start 136.07246 90.639813) (end 137.47246 89.239813) (width 0.5) (layer "F.Cu") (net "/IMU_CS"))
 (segment (start 136.07246 97.36184) (end 136.07246 90.639813) (width 0.5) (layer "F.Cu") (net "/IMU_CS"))
 (segment (start 164.488187 98.071813) (end 136.782433 98.071813) (width 0.5) (layer "F.Cu") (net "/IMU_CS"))
 (segment (start 165.86 96.7) (end 164.488187 98.071813) (width 0.5) (layer "F.Cu") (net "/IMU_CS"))
 (segment (start 136.782433 98.071813) (end 136.07246 97.36184) (width 0.5) (layer "F.Cu") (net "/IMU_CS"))
 (segment (start 163.848187 103.151813) (end 136.782433 103.151813) (width 0.5) (layer "F.Cu") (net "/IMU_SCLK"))
 (segment (start 134 89.098273) (end 136.39846 86.699813) (width 0.5) (layer "F.Cu") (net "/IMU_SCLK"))
 (segment (start 134 100.36938) (end 134 89.098273) (width 0.5) (layer "F.Cu") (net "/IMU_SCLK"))
 (segment (start 136.782433 103.151813) (end 134 100.36938) (width 0.5) (layer "F.Cu") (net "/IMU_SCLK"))
 (segment (start 169 98) (end 163.848187 103.151813) (width 0.5) (layer "F.Cu") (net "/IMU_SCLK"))
 (segment (start 136.39846 86.699813) (end 137.47246 86.699813) (width 0.5) (layer "F.Cu") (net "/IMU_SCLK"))
 (segment (start 165.86 91.62) (end 169 94.76) (width 0.5) (layer "F.Cu") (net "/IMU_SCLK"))
 (segment (start 169 94.76) (end 169 98) (width 0.5) (layer "F.Cu") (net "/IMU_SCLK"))
 (segment (start 167.21 97.259189) (end 163.857376 100.611813) (width 0.5) (layer "F.Cu") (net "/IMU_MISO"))
 (segment (start 163.857376 100.611813) (end 136.782433 100.611813) (width 0.5) (layer "F.Cu") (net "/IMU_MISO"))
 (segment (start 136.782433 100.611813) (end 135.37246 99.20184) (width 0.5) (layer "F.Cu") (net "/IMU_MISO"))
 (segment (start 139 85.687353) (end 137.47246 84.159813) (width 0.5) (layer "F.Cu") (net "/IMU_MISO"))
 (segment (start 136.782433 87.911813) (end 138.162487 87.911813) (width 0.5) (layer "F.Cu") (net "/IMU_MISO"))
 (segment (start 138.162487 87.911813) (end 139 87.0743) (width 0.5) (layer "F.Cu") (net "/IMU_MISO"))
 (segment (start 135.37246 99.20184) (end 135.37246 89.321786) (width 0.5) (layer "F.Cu") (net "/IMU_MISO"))
 (segment (start 167.21 95.51) (end 167.21 97.259189) (width 0.5) (layer "F.Cu") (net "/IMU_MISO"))
 (segment (start 135.37246 89.321786) (end 136.782433 87.911813) (width 0.5) (layer "F.Cu") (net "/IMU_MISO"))
 (segment (start 139 87.0743) (end 139 85.687353) (width 0.5) (layer "F.Cu") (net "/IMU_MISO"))
 (segment (start 165.86 94.16) (end 167.21 95.51) (width 0.5) (layer "F.Cu") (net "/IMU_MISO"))
 (segment (start 148.92 71) (end 147.132187 72.787813) (width 0.5) (layer "F.Cu") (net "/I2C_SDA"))
 (segment (start 136.782433 72.787813) (end 136.07246 73.497786) (width 0.5) (layer "F.Cu") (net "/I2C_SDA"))
 (segment (start 136.07246 73.497786) (end 136.07246 80.219813) (width 0.5) (layer "F.Cu") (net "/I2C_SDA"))
 (segment (start 147.132187 72.787813) (end 136.782433 72.787813) (width 0.5) (layer "F.Cu") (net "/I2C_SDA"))
 (segment (start 136.07246 80.219813) (end 137.47246 81.619813) (width 0.5) (layer "F.Cu") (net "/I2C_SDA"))
 (segment (start 148.92 66) (end 148.92 71) (width 0.5) (layer "F.Cu") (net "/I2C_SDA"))
 (segment (start 148.460187 73.999813) (end 137.47246 73.999813) (width 0.5) (layer "F.Cu") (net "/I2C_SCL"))
 (segment (start 151.46 71) (end 148.460187 73.999813) (width 0.5) (layer "F.Cu") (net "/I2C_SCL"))
 (segment (start 151.46 66) (end 151.46 71) (width 0.5) (layer "F.Cu") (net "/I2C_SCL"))
 (segment (start 136.39846 71.459813) (end 137.47246 71.459813) (width 0.5) (layer "F.Cu") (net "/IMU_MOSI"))
 (segment (start 135.37246 82.37246) (end 135.37246 72.485813) (width 0.5) (layer "F.Cu") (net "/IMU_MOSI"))
 (segment (start 135.831813 82.831813) (end 135.37246 82.37246) (width 0.5) (layer "F.Cu") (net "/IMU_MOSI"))
 (segment (start 138.87246 82.12184) (end 138.162487 82.831813) (width 0.5) (layer "F.Cu") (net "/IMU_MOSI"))
 (segment (start 135.37246 72.485813) (end 136.39846 71.459813) (width 0.5) (layer "F.Cu") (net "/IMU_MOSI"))
 (segment (start 165.86 89.08) (end 158.90184 82.12184) (width 0.5) (layer "F.Cu") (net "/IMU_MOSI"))
 (segment (start 138.162487 82.831813) (end 135.831813 82.831813) (width 0.5) (layer "F.Cu") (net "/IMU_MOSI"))
 (segment (start 158.90184 82.12184) (end 138.87246 82.12184) (width 0.5) (layer "F.Cu") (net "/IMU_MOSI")))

